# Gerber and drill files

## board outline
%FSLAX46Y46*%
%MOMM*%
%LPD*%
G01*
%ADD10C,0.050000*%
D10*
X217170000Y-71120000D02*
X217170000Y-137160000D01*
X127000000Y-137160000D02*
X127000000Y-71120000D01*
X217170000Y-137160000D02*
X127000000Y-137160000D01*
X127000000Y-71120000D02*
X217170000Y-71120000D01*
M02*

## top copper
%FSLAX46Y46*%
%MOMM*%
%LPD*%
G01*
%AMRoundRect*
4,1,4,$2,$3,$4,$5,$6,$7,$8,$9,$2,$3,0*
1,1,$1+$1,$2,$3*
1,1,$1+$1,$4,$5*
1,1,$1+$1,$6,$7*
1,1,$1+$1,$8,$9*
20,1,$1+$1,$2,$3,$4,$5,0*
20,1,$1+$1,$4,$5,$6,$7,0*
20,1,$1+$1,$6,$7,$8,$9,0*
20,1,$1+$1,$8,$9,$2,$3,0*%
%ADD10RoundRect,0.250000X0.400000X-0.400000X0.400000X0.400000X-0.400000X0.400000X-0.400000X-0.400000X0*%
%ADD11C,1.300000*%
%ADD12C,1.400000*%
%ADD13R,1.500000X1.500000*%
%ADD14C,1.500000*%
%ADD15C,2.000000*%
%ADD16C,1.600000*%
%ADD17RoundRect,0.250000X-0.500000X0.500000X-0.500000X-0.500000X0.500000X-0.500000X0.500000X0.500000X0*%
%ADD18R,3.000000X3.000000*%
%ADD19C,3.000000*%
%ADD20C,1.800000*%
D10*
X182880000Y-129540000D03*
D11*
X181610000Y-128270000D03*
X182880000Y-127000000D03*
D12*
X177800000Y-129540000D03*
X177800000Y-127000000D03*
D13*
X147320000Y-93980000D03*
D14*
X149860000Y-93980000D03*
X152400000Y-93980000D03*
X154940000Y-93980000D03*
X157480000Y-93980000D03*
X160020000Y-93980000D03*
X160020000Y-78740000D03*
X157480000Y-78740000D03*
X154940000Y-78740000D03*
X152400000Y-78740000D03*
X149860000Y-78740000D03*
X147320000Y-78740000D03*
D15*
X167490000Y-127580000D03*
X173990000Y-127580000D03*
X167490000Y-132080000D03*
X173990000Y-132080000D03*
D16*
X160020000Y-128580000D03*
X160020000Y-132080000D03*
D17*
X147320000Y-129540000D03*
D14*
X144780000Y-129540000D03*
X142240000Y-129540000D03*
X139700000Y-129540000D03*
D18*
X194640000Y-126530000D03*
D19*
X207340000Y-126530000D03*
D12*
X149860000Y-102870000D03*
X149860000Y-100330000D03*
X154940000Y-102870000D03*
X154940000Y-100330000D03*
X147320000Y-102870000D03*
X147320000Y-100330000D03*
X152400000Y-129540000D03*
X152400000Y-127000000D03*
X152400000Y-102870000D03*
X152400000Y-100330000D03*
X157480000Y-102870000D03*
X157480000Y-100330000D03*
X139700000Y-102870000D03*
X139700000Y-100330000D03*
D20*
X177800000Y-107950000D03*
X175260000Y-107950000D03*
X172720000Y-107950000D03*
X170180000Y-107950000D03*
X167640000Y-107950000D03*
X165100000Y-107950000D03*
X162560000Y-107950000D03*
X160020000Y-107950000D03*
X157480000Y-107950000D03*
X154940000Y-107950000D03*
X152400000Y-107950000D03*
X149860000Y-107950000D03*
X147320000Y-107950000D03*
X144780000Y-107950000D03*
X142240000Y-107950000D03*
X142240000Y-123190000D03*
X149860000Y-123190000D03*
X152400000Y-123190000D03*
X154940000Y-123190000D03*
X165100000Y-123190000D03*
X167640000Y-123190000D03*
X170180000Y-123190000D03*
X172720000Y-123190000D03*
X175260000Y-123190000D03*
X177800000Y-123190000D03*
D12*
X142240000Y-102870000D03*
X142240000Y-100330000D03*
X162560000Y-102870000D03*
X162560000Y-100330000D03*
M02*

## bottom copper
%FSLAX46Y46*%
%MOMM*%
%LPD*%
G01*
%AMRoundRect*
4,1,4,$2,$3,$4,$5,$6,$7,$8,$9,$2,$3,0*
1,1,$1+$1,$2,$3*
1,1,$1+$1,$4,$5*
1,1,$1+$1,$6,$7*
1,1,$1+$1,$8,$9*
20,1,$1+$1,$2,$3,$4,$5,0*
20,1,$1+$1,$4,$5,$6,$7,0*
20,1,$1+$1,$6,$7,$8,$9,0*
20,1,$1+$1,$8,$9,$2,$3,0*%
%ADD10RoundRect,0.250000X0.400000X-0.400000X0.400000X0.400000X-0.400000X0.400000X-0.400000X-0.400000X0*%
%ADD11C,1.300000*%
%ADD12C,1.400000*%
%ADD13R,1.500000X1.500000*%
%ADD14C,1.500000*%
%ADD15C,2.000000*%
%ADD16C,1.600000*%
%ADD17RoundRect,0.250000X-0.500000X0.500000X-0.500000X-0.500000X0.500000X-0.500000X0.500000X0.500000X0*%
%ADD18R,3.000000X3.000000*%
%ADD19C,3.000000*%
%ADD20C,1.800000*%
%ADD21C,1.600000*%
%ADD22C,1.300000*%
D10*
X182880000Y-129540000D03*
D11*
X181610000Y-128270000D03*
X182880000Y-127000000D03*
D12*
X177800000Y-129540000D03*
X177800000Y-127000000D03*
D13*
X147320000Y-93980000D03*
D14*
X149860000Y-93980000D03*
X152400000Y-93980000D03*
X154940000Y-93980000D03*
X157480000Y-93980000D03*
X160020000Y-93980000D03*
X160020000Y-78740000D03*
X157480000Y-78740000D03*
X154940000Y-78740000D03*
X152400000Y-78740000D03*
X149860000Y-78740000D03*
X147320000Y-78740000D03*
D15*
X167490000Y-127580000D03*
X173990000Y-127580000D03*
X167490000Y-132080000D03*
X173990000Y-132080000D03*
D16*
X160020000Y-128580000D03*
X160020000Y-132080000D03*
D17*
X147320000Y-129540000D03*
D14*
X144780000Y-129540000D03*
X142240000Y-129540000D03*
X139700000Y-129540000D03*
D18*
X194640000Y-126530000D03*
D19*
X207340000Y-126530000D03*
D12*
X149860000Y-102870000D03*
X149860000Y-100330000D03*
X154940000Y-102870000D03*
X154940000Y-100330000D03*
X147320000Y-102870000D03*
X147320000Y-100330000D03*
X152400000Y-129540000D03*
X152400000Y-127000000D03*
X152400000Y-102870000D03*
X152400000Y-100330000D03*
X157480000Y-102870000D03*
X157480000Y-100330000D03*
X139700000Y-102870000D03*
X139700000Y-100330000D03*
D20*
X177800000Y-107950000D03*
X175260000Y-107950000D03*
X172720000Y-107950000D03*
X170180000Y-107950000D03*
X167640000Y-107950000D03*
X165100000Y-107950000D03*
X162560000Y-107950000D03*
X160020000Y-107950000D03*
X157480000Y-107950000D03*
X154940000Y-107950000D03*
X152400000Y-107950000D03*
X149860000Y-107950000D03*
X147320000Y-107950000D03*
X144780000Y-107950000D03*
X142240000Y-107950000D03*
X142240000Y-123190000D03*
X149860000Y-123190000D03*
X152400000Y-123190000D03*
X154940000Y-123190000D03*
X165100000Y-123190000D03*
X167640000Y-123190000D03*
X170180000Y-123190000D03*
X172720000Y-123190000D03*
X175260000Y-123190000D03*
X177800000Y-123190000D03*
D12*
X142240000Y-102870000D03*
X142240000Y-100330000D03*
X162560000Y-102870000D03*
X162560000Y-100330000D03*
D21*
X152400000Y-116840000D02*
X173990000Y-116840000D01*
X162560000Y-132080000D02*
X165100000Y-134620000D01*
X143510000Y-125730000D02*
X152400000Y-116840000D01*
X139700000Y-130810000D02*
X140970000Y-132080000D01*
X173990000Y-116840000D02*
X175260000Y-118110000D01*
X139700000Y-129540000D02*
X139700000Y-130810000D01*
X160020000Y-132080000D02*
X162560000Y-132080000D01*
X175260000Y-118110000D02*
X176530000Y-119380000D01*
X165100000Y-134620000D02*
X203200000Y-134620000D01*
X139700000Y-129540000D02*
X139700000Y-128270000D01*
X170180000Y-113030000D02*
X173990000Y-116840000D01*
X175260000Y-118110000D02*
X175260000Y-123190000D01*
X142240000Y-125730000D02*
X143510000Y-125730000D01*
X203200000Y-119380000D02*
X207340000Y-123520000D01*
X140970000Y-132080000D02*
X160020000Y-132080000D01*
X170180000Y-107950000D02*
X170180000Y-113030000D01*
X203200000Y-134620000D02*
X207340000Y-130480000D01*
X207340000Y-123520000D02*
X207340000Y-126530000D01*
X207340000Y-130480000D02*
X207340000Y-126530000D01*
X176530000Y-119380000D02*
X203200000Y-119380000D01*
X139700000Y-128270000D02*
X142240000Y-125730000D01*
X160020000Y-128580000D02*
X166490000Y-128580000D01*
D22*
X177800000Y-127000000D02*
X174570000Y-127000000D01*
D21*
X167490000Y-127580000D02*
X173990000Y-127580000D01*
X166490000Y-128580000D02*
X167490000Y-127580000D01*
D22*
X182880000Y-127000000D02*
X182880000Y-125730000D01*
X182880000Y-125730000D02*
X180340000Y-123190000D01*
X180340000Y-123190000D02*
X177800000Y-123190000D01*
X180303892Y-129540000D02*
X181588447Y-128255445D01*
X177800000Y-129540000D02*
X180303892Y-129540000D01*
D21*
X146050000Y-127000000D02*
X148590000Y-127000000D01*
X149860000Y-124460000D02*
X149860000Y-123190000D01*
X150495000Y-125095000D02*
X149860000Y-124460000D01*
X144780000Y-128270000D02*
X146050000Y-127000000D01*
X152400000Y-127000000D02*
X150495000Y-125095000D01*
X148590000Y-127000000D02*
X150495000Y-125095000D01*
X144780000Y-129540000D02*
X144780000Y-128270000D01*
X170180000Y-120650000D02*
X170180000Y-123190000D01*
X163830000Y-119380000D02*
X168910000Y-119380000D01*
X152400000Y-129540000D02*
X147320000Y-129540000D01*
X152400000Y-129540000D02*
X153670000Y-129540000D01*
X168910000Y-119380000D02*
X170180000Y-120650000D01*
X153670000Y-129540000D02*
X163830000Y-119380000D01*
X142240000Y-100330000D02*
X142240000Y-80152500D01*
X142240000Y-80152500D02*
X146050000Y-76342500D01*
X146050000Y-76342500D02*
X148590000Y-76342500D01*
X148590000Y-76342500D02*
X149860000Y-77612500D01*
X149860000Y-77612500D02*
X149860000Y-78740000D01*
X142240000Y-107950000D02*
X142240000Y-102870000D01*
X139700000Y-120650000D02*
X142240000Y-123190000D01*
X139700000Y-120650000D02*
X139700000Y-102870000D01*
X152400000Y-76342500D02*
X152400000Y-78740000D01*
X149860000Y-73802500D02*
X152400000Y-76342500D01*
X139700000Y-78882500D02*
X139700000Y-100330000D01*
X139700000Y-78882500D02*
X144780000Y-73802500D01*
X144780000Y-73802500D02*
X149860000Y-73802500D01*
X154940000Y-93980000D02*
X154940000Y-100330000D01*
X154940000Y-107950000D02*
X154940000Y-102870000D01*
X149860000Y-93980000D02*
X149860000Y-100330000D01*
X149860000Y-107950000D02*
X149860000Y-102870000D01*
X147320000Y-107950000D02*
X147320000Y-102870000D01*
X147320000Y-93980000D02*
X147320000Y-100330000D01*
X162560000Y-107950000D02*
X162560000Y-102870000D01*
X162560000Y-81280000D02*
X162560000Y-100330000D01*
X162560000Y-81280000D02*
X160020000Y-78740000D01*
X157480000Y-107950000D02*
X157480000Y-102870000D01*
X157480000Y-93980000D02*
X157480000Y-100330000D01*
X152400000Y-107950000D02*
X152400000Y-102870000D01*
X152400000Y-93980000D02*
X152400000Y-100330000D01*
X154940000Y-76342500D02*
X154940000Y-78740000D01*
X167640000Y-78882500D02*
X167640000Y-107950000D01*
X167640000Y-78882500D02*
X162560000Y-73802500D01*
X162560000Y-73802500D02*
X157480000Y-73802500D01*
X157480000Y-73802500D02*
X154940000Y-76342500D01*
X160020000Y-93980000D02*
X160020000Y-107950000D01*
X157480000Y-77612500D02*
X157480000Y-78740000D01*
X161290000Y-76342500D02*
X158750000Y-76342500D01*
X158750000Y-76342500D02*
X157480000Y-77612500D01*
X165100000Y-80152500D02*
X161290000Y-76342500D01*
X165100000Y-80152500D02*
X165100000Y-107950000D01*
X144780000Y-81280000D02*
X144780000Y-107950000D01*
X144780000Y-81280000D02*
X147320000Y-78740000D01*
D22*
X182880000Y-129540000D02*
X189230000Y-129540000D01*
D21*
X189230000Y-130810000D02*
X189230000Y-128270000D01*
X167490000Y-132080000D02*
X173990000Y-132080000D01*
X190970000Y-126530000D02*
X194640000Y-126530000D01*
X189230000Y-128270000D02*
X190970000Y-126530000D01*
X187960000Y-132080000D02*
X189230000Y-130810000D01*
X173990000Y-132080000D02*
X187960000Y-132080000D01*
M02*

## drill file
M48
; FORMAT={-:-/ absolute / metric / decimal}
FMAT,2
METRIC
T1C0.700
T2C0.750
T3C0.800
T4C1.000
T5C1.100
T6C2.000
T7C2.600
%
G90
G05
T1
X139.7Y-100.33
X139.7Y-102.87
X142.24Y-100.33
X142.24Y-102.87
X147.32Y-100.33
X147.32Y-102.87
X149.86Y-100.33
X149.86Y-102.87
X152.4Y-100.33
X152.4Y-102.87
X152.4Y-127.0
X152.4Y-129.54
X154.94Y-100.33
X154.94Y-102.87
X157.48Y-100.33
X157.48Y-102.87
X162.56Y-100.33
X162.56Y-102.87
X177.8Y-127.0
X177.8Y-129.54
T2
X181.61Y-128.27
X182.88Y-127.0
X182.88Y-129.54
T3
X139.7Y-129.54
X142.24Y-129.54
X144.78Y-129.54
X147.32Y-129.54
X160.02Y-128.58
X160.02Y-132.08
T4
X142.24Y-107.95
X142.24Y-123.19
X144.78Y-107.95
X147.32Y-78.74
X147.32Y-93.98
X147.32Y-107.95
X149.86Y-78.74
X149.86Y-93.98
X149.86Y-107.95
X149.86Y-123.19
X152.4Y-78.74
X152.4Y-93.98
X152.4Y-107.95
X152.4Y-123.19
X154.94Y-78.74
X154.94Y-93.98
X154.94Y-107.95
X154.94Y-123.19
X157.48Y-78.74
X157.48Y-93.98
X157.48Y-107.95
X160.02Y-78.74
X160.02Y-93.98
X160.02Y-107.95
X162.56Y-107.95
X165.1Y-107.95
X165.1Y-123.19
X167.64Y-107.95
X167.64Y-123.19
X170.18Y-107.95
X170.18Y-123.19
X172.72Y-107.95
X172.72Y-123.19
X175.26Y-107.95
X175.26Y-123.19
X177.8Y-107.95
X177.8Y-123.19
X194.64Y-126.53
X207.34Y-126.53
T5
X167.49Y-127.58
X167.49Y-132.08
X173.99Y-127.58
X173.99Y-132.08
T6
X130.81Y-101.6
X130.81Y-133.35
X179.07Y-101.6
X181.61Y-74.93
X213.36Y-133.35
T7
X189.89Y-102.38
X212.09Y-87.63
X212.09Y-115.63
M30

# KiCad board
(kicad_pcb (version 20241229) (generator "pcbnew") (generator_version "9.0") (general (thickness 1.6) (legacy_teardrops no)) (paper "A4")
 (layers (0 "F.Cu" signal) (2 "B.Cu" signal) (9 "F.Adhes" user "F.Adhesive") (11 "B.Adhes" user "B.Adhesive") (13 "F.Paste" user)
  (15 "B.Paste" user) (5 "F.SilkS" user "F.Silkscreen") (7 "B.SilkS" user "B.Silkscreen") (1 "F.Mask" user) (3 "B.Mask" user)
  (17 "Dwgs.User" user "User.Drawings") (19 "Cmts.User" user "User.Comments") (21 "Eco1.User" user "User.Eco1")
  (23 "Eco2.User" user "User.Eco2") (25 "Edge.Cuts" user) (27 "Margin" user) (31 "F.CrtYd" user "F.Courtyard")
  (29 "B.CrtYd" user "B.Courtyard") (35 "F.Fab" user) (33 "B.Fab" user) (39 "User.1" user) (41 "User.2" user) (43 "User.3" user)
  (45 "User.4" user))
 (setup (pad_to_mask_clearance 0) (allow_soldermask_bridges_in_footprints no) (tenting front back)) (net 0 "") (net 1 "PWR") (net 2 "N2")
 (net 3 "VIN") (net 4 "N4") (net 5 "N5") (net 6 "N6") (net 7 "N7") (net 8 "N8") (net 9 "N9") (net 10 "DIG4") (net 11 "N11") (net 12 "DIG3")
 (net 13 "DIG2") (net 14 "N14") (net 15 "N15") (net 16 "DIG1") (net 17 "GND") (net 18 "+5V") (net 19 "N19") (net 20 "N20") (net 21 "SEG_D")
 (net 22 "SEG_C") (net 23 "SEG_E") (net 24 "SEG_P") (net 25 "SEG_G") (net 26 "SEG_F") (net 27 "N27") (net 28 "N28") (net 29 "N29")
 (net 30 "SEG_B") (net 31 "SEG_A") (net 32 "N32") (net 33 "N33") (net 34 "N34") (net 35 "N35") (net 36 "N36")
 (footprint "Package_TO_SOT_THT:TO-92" (layer "F.Cu") (at 182.88 129.54 90)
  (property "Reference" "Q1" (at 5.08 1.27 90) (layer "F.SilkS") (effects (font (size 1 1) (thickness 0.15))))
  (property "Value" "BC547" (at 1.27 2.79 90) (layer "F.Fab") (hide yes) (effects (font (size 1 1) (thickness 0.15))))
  (pad "1" thru_hole roundrect (at 0 0 90) (size 1.3 1.3) (drill 0.75) (layers "*.Cu" "*.Mask") (remove_unused_layers no)
   (roundrect_rratio 0.1923076923) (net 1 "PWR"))
  (pad "2" thru_hole circle (at 1.27 -1.27 90) (size 1.3 1.3) (drill 0.75) (layers "*.Cu" "*.Mask") (remove_unused_layers no) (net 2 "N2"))
  (pad "3" thru_hole circle (at 2.54 0 90) (size 1.3 1.3) (drill 0.75) (layers "*.Cu" "*.Mask") (remove_unused_layers no) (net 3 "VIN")))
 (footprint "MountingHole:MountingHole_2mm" (layer "F.Cu") (at 130.81 133.35)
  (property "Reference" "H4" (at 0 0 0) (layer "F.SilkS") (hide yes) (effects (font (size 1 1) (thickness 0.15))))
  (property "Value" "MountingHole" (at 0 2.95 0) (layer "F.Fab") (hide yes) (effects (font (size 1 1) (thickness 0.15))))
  (pad "" np_thru_hole circle (at 0 0) (size 2 2) (drill 2) (layers "*.Cu" "*.Mask")))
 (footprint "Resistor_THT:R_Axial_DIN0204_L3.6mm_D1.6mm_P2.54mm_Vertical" (layer "F.Cu") (at 177.8 129.54 90)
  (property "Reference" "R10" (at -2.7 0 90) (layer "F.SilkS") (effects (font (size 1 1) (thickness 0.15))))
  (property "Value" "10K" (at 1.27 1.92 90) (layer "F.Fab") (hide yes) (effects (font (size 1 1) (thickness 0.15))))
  (pad "1" thru_hole circle (at 0 0 90) (size 1.4 1.4) (drill 0.7) (layers "*.Cu" "*.Mask") (remove_unused_layers no) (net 2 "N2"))
  (pad "2" thru_hole circle (at 2.54 0 90) (size 1.4 1.4) (drill 0.7) (layers "*.Cu" "*.Mask") (remove_unused_layers no) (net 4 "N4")))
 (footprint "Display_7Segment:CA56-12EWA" (layer "F.Cu") (at 147.32 93.98 90)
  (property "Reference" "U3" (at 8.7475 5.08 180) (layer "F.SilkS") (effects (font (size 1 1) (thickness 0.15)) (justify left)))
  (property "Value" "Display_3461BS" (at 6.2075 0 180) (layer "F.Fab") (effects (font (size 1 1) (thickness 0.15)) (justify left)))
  (pad "1" thru_hole rect (at 0 0 90) (size 1.5 1.5) (drill 1) (layers "*.Cu" "*.Mask") (remove_unused_layers no) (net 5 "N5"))
  (pad "2" thru_hole circle (at 0 2.54 90) (size 1.5 1.5) (drill 1) (layers "*.Cu" "*.Mask") (remove_unused_layers no) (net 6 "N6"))
  (pad "3" thru_hole circle (at 0 5.08 90) (size 1.5 1.5) (drill 1) (layers "*.Cu" "*.Mask") (remove_unused_layers no) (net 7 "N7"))
  (pad "4" thru_hole circle (at 0 7.62 90) (size 1.5 1.5) (drill 1) (layers "*.Cu" "*.Mask") (remove_unused_layers no) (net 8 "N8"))
  (pad "5" thru_hole circle (at 0 10.16 90) (size 1.5 1.5) (drill 1) (layers "*.Cu" "*.Mask") (remove_unused_layers no) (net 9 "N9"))
  (pad "6" thru_hole circle (at 0 12.7 90) (size 1.5 1.5) (drill 1) (layers "*.Cu" "*.Mask") (remove_unused_layers no) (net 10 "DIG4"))
  (pad "7" thru_hole circle (at 15.24 12.7 90) (size 1.5 1.5) (drill 1) (layers "*.Cu" "*.Mask") (remove_unused_layers no) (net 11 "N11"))
  (pad "8" thru_hole circle (at 15.24 10.16 90) (size 1.5 1.5) (drill 1) (layers "*.Cu" "*.Mask") (remove_unused_layers no) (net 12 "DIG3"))
  (pad "9" thru_hole circle (at 15.24 7.62 90) (size 1.5 1.5) (drill 1) (layers "*.Cu" "*.Mask") (remove_unused_layers no) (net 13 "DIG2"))
  (pad "10" thru_hole circle (at 15.24 5.08 90) (size 1.5 1.5) (drill 1) (layers "*.Cu" "*.Mask") (remove_unused_layers no) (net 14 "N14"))
  (pad "11" thru_hole circle (at 15.24 2.54 90) (size 1.5 1.5) (drill 1) (layers "*.Cu" "*.Mask") (remove_unused_layers no) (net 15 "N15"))
  (pad "12" thru_hole circle (at 15.24 0 90) (size 1.5 1.5) (drill 1) (layers "*.Cu" "*.Mask") (remove_unused_layers no) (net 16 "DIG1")))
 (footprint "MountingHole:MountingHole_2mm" (layer "F.Cu") (at 130.81 101.6)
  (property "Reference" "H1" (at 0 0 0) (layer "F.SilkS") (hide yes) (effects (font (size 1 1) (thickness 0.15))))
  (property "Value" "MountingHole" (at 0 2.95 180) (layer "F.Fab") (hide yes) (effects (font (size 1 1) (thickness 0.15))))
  (pad "" np_thru_hole circle (at 0 0) (size 2 2) (drill 2) (layers "*.Cu" "*.Mask")))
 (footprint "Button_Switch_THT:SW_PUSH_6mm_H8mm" (layer "F.Cu") (at 167.49 127.58)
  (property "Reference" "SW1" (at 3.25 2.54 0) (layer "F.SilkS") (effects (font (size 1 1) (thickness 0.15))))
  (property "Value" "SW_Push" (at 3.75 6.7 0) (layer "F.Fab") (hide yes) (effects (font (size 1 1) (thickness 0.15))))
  (pad "1" thru_hole circle (at 0 0 90) (size 2 2) (drill 1.1) (layers "*.Cu" "*.Mask") (remove_unused_layers no) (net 4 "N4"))
  (pad "1" thru_hole circle (at 6.5 0 90) (size 2 2) (drill 1.1) (layers "*.Cu" "*.Mask") (remove_unused_layers no) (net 4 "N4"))
  (pad "2" thru_hole circle (at 0 4.5 90) (size 2 2) (drill 1.1) (layers "*.Cu" "*.Mask") (remove_unused_layers no) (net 1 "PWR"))
  (pad "2" thru_hole circle (at 6.5 4.5 90) (size 2 2) (drill 1.1) (layers "*.Cu" "*.Mask") (remove_unused_layers no) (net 1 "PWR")))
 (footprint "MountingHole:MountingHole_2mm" (layer "F.Cu") (at 179.07 101.6)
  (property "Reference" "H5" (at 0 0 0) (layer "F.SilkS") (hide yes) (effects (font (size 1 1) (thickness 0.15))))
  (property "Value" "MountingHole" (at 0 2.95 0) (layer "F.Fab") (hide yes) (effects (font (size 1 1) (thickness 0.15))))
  (pad "" np_thru_hole circle (at 0 0) (size 2 2) (drill 2) (layers "*.Cu" "*.Mask")))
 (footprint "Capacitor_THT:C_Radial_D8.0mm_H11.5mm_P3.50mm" (layer "F.Cu") (at 160.02 128.58 -90)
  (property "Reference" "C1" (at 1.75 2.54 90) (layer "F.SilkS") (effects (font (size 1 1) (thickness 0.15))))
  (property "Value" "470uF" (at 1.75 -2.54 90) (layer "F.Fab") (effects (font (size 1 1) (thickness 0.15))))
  (pad "1" thru_hole circle (at 0 0 270) (size 1.6 1.6) (drill 0.8) (layers "*.Cu" "*.Mask") (remove_unused_layers no) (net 4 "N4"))
  (pad "2" thru_hole circle (at 3.5 0 270) (size 1.6 1.6) (drill 0.8) (layers "*.Cu" "*.Mask") (remove_unused_layers no) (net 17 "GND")))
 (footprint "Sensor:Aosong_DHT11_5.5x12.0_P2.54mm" (layer "F.Cu") (at 147.32 129.54 -90)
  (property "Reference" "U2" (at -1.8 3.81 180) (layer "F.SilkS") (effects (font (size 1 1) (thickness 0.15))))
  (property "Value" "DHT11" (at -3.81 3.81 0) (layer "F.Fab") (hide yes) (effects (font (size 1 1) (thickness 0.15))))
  (pad "1" thru_hole roundrect (at 0 0 270) (size 1.5 1.5) (drill 0.8) (layers "*.Cu" "*.Mask") (remove_unused_layers no)
   (roundrect_rratio 0.1666666667) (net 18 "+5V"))
  (pad "2" thru_hole circle (at 0 2.54 270) (size 1.5 1.5) (drill 0.8) (layers "*.Cu" "*.Mask") (remove_unused_layers no) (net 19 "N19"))
  (pad "3" thru_hole circle (at 0 5.08 270) (size 1.5 1.5) (drill 0.8) (layers "*.Cu" "*.Mask") (remove_unused_layers no) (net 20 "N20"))
  (pad "4" thru_hole circle (at 0 7.62 270) (size 1.5 1.5) (drill 0.8) (layers "*.Cu" "*.Mask") (remove_unused_layers no) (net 17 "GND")))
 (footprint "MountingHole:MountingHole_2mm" (layer "F.Cu") (at 213.36 133.35)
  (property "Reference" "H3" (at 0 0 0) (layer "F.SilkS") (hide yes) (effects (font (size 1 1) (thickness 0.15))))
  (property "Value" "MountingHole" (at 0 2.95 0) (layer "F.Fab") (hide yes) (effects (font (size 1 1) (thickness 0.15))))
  (pad "" np_thru_hole circle (at 0 0) (size 2 2) (drill 2) (layers "*.Cu" "*.Mask")))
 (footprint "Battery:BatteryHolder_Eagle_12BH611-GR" (layer "F.Cu") (at 194.64 126.53 -90)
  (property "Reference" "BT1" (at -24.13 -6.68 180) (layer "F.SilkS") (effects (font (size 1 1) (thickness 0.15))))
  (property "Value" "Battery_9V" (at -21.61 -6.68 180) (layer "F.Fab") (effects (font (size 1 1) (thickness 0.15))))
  (pad "" np_thru_hole circle (at -38.9 -17.45 270) (size 2.6 2.6) (drill 2.6) (layers "*.Cu" "*.Mask"))
  (pad "" np_thru_hole circle (at -24.15 4.75 270) (size 2.6 2.6) (drill 2.6) (layers "*.Cu" "*.Mask"))
  (pad "" np_thru_hole circle (at -10.9 -17.45 270) (size 2.6 2.6) (drill 2.6) (layers "*.Cu" "*.Mask"))
  (pad "1" thru_hole rect (at 0 0 270) (size 3 3) (drill 1) (layers "*.Cu" "*.Mask") (remove_unused_layers no) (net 1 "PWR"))
  (pad "2" thru_hole circle (at 0 -12.7 270) (size 3 3) (drill 1) (layers "*.Cu" "*.Mask") (remove_unused_layers no) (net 17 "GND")))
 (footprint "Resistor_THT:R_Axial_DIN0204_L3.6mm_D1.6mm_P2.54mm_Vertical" (layer "F.Cu") (at 149.86 102.87 90)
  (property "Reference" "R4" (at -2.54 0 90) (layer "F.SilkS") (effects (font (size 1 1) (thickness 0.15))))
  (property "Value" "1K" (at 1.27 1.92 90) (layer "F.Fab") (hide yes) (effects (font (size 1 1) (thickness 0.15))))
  (pad "1" thru_hole circle (at 0 0 90) (size 1.4 1.4) (drill 0.7) (layers "*.Cu" "*.Mask") (remove_unused_layers no) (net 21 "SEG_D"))
  (pad "2" thru_hole circle (at 2.54 0 90) (size 1.4 1.4) (drill 0.7) (layers "*.Cu" "*.Mask") (remove_unused_layers no) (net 6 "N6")))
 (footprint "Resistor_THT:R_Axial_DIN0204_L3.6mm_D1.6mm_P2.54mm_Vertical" (layer "F.Cu") (at 154.94 102.87 90)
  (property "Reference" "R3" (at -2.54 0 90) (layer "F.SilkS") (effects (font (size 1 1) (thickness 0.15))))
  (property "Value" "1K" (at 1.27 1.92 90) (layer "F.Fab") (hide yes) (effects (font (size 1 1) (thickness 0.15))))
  (pad "1" thru_hole circle (at 0 0 90) (size 1.4 1.4) (drill 0.7) (layers "*.Cu" "*.Mask") (remove_unused_layers no) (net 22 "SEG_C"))
  (pad "2" thru_hole circle (at 2.54 0 90) (size 1.4 1.4) (drill 0.7) (layers "*.Cu" "*.Mask") (remove_unused_layers no) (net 8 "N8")))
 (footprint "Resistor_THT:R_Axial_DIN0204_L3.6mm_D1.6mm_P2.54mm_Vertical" (layer "F.Cu") (at 147.32 102.87 90)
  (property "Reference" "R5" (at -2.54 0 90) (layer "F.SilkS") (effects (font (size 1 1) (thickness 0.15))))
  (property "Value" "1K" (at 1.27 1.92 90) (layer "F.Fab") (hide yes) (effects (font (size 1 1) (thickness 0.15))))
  (pad "1" thru_hole circle (at 0 0 90) (size 1.4 1.4) (drill 0.7) (layers "*.Cu" "*.Mask") (remove_unused_layers no) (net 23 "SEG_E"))
  (pad "2" thru_hole circle (at 2.54 0 90) (size 1.4 1.4) (drill 0.7) (layers "*.Cu" "*.Mask") (remove_unused_layers no) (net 5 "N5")))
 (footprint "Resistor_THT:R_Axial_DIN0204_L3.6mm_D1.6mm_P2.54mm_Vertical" (layer "F.Cu") (at 152.4 129.54 90)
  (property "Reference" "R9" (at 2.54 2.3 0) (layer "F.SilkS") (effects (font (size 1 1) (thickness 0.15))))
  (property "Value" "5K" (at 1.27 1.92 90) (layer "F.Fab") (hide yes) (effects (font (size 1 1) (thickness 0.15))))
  (pad "1" thru_hole circle (at 0 0 90) (size 1.4 1.4) (drill 0.7) (layers "*.Cu" "*.Mask") (remove_unused_layers no) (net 18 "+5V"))
  (pad "2" thru_hole circle (at 2.54 0 90) (size 1.4 1.4) (drill 0.7) (layers "*.Cu" "*.Mask") (remove_unused_layers no) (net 19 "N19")))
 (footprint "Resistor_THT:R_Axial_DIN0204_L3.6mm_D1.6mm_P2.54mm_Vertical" (layer "F.Cu") (at 152.4 102.87 90)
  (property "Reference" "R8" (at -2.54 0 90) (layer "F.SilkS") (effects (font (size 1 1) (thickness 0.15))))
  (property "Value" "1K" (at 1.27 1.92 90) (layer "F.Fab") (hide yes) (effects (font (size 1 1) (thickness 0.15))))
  (pad "1" thru_hole circle (at 0 0 90) (size 1.4 1.4) (drill 0.7) (layers "*.Cu" "*.Mask") (remove_unused_layers no) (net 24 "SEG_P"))
  (pad "2" thru_hole circle (at 2.54 0 90) (size 1.4 1.4) (drill 0.7) (layers "*.Cu" "*.Mask") (remove_unused_layers no) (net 7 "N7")))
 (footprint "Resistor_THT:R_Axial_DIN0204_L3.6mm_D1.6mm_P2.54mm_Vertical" (layer "F.Cu") (at 157.48 102.87 90)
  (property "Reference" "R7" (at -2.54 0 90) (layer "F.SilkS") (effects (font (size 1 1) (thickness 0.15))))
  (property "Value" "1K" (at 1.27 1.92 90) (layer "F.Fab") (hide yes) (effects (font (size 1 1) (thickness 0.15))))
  (pad "1" thru_hole circle (at 0 0 90) (size 1.4 1.4) (drill 0.7) (layers "*.Cu" "*.Mask") (remove_unused_layers no) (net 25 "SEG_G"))
  (pad "2" thru_hole circle (at 2.54 0 90) (size 1.4 1.4) (drill 0.7) (layers "*.Cu" "*.Mask") (remove_unused_layers no) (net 9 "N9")))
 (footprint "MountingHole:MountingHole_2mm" (layer "F.Cu") (at 181.61 74.93)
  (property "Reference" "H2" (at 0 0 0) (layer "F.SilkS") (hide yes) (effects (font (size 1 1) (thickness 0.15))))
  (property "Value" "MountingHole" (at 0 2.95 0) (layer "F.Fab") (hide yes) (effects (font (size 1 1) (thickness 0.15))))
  (pad "" np_thru_hole circle (at 0 0) (size 2 2) (drill 2) (layers "*.Cu" "*.Mask")))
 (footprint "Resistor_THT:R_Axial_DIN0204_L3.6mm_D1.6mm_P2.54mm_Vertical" (layer "F.Cu") (at 139.7 102.87 90)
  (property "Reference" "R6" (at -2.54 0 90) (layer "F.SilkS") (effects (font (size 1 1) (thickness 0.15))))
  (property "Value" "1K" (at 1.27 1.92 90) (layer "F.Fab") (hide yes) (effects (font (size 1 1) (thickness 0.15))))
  (pad "1" thru_hole circle (at 0 0 90) (size 1.4 1.4) (drill 0.7) (layers "*.Cu" "*.Mask") (remove_unused_layers no) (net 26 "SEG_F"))
  (pad "2" thru_hole circle (at 2.54 0 90) (size 1.4 1.4) (drill 0.7) (layers "*.Cu" "*.Mask") (remove_unused_layers no) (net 14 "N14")))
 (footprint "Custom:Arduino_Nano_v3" (layer "F.Cu") (at 177.8 107.95 -90)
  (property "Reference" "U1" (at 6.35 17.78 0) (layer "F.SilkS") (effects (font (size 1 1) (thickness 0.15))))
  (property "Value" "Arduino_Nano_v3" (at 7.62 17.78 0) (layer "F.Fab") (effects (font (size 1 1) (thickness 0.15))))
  (pad "1" thru_hole circle (at 0 0 270) (size 1.8 1.8) (drill 1) (layers "*.Cu" "*.Mask") (remove_unused_layers no) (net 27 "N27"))
  (pad "2" thru_hole circle (at 0 2.54 270) (size 1.8 1.8) (drill 1) (layers "*.Cu" "*.Mask") (remove_unused_layers no) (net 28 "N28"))
  (pad "3" thru_hole circle (at 0 5.08 270) (size 1.8 1.8) (drill 1) (layers "*.Cu" "*.Mask") (remove_unused_layers no) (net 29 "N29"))
  (pad "4" thru_hole circle (at 0 7.62 270) (size 1.8 1.8) (drill 1) (layers "*.Cu" "*.Mask") (remove_unused_layers no) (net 17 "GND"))
  (pad "5" thru_hole circle (at 0 10.16 270) (size 1.8 1.8) (drill 1) (layers "*.Cu" "*.Mask") (remove_unused_layers no) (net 13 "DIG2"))
  (pad "6" thru_hole circle (at 0 12.7 270) (size 1.8 1.8) (drill 1) (layers "*.Cu" "*.Mask") (remove_unused_layers no) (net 12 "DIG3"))
  (pad "7" thru_hole circle (at 0 15.24 270) (size 1.8 1.8) (drill 1) (layers "*.Cu" "*.Mask") (remove_unused_layers no) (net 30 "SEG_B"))
  (pad "8" thru_hole circle (at 0 17.78 270) (size 1.8 1.8) (drill 1) (layers "*.Cu" "*.Mask") (remove_unused_layers no) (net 10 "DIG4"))
  (pad "9" thru_hole circle (at 0 20.32 270) (size 1.8 1.8) (drill 1) (layers "*.Cu" "*.Mask") (remove_unused_layers no) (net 25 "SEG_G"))
  (pad "10" thru_hole circle (at 0 22.86 270) (size 1.8 1.8) (drill 1) (layers "*.Cu" "*.Mask") (remove_unused_layers no) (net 22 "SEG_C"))
  (pad "11" thru_hole circle (at 0 25.4 270) (size 1.8 1.8) (drill 1) (layers "*.Cu" "*.Mask") (remove_unused_layers no) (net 24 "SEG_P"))
  (pad "12" thru_hole circle (at 0 27.94 270) (size 1.8 1.8) (drill 1) (layers "*.Cu" "*.Mask") (remove_unused_layers no) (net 21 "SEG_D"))
  (pad "13" thru_hole circle (at 0 30.48 270) (size 1.8 1.8) (drill 1) (layers "*.Cu" "*.Mask") (remove_unused_layers no) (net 23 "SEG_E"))
  (pad "14" thru_hole circle (at 0 33.02 270) (size 1.8 1.8) (drill 1) (layers "*.Cu" "*.Mask") (remove_unused_layers no) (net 16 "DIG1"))
  (pad "15" thru_hole circle (at 0 35.56 270) (size 1.8 1.8) (drill 1) (layers "*.Cu" "*.Mask") (remove_unused_layers no) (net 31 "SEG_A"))
  (pad "16" thru_hole circle (at 15.24 35.56 270) (size 1.8 1.8) (drill 1) (layers "*.Cu" "*.Mask") (remove_unused_layers no)
   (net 26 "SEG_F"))
  (pad "19" thru_hole circle (at 15.24 27.94 270) (size 1.8 1.8) (drill 1) (layers "*.Cu" "*.Mask") (remove_unused_layers no) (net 19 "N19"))
  (pad "20" thru_hole circle (at 15.24 25.4 270) (size 1.8 1.8) (drill 1) (layers "*.Cu" "*.Mask") (remove_unused_layers no) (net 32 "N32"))
  (pad "21" thru_hole circle (at 15.24 22.86 270) (size 1.8 1.8) (drill 1) (layers "*.Cu" "*.Mask") (remove_unused_layers no) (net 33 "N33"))
  (pad "25" thru_hole circle (at 15.24 12.7 270) (size 1.8 1.8) (drill 1) (layers "*.Cu" "*.Mask") (remove_unused_layers no) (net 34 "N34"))
  (pad "26" thru_hole circle (at 15.24 10.16 270) (size 1.8 1.8) (drill 1) (layers "*.Cu" "*.Mask") (remove_unused_layers no) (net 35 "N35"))
  (pad "27" thru_hole circle (at 15.24 7.62 270) (size 1.8 1.8) (drill 1) (layers "*.Cu" "*.Mask") (remove_unused_layers no) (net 18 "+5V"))
  (pad "28" thru_hole circle (at 15.24 5.08 270) (size 1.8 1.8) (drill 1) (layers "*.Cu" "*.Mask") (remove_unused_layers no) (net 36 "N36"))
  (pad "29" thru_hole circle (at 15.24 2.54 270) (size 1.8 1.8) (drill 1) (layers "*.Cu" "*.Mask") (remove_unused_layers no) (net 17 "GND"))
  (pad "30" thru_hole circle (at 15.24 0 270) (size 1.8 1.8) (drill 1) (layers "*.Cu" "*.Mask") (remove_unused_layers no) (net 3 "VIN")))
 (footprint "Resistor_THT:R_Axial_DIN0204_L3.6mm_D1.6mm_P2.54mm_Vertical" (layer "F.Cu") (at 142.24 102.87 90)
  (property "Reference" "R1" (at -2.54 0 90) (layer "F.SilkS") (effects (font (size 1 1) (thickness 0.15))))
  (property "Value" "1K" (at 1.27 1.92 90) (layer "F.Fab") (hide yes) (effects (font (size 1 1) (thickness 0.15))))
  (pad "1" thru_hole circle (at 0 0 90) (size 1.4 1.4) (drill 0.7) (layers "*.Cu" "*.Mask") (remove_unused_layers no) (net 31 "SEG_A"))
  (pad "2" thru_hole circle (at 2.54 0 90) (size 1.4 1.4) (drill 0.7) (layers "*.Cu" "*.Mask") (remove_unused_layers no) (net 15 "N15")))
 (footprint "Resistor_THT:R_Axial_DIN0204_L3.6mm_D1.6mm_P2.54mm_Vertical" (layer "F.Cu") (at 162.56 102.87 90)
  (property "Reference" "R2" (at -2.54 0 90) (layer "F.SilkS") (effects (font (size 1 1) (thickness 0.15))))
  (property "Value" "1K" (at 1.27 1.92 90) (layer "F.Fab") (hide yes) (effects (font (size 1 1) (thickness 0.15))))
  (pad "1" thru_hole circle (at 0 0 90) (size 1.4 1.4) (drill 0.7) (layers "*.Cu" "*.Mask") (remove_unused_layers no) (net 30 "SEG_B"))
  (pad "2" thru_hole circle (at 2.54 0 90) (size 1.4 1.4) (drill 0.7) (layers "*.Cu" "*.Mask") (remove_unused_layers no) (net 11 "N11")))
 (gr_line (start 217.17 71.12) (end 217.17 137.16) (stroke (width 0.05) (type default)) (layer "Edge.Cuts"))
 (gr_line (start 127 137.16) (end 127 71.12) (stroke (width 0.05) (type default)) (layer "Edge.Cuts"))
 (gr_line (start 217.17 137.16) (end 127 137.16) (stroke (width 0.05) (type default)) (layer "Edge.Cuts"))
 (gr_line (start 127 71.12) (end 217.17 71.12) (stroke (width 0.05) (type default)) (layer "Edge.Cuts"))
 (segment (start 152.4 116.84) (end 173.99 116.84) (width 1.6) (layer "B.Cu") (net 17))
 (segment (start 162.56 132.08) (end 165.1 134.62) (width 1.6) (layer "B.Cu") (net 17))
 (segment (start 143.51 125.73) (end 152.4 116.84) (width 1.6) (layer "B.Cu") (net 17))
 (segment (start 139.7 130.81) (end 140.97 132.08) (width 1.6) (layer "B.Cu") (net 17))
 (segment (start 173.99 116.84) (end 175.26 118.11) (width 1.6) (layer "B.Cu") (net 17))
 (segment (start 139.7 129.54) (end 139.7 130.81) (width 1.6) (layer "B.Cu") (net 17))
 (segment (start 160.02 132.08) (end 162.56 132.08) (width 1.6) (layer "B.Cu") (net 17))
 (segment (start 175.26 118.11) (end 176.53 119.38) (width 1.6) (layer "B.Cu") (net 17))
 (segment (start 165.1 134.62) (end 203.2 134.62) (width 1.6) (layer "B.Cu") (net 17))
 (segment (start 139.7 129.54) (end 139.7 128.27) (width 1.6) (layer "B.Cu") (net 17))
 (segment (start 170.18 113.03) (end 173.99 116.84) (width 1.6) (layer "B.Cu") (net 17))
 (segment (start 175.26 118.11) (end 175.26 123.19) (width 1.6) (layer "B.Cu") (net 17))
 (segment (start 142.24 125.73) (end 143.51 125.73) (width 1.6) (layer "B.Cu") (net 17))
 (segment (start 203.2 119.38) (end 207.34 123.52) (width 1.6) (layer "B.Cu") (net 17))
 (segment (start 140.97 132.08) (end 160.02 132.08) (width 1.6) (layer "B.Cu") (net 17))
 (segment (start 170.18 107.95) (end 170.18 113.03) (width 1.6) (layer "B.Cu") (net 17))
 (segment (start 203.2 134.62) (end 207.34 130.48) (width 1.6) (layer "B.Cu") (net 17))
 (segment (start 207.34 123.52) (end 207.34 126.53) (width 1.6) (layer "B.Cu") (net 17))
 (segment (start 207.34 130.48) (end 207.34 126.53) (width 1.6) (layer "B.Cu") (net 17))
 (segment (start 176.53 119.38) (end 203.2 119.38) (width 1.6) (layer "B.Cu") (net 17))
 (segment (start 139.7 128.27) (end 142.24 125.73) (width 1.6) (layer "B.Cu") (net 17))
 (segment (start 160.02 128.58) (end 166.49 128.58) (width 1.6) (layer "B.Cu") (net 4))
 (segment (start 177.8 127) (end 174.57 127) (width 1.3) (layer "B.Cu") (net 4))
 (segment (start 167.49 127.58) (end 173.99 127.58) (width 1.6) (layer "B.Cu") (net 4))
 (segment (start 166.49 128.58) (end 167.49 127.58) (width 1.6) (layer "B.Cu") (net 4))
 (segment (start 182.88 127) (end 182.88 125.73) (width 1.3) (layer "B.Cu") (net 3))
 (segment (start 182.88 125.73) (end 180.34 123.19) (width 1.3) (layer "B.Cu") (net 3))
 (segment (start 180.34 123.19) (end 177.8 123.19) (width 1.3) (layer "B.Cu") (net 3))
 (segment (start 180.303892 129.54) (end 181.588447 128.255445) (width 1.3) (layer "B.Cu") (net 2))
 (segment (start 177.8 129.54) (end 180.303892 129.54) (width 1.3) (layer "B.Cu") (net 2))
 (segment (start 146.05 127) (end 148.59 127) (width 1.6) (layer "B.Cu") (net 19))
 (segment (start 149.86 124.46) (end 149.86 123.19) (width 1.6) (layer "B.Cu") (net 19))
 (segment (start 150.495 125.095) (end 149.86 124.46) (width 1.6) (layer "B.Cu") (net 19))
 (segment (start 144.78 128.27) (end 146.05 127) (width 1.6) (layer "B.Cu") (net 19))
 (segment (start 152.4 127) (end 150.495 125.095) (width 1.6) (layer "B.Cu") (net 19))
 (segment (start 148.59 127) (end 150.495 125.095) (width 1.6) (layer "B.Cu") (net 19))
 (segment (start 144.78 129.54) (end 144.78 128.27) (width 1.6) (layer "B.Cu") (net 19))
 (segment (start 170.18 120.65) (end 170.18 123.19) (width 1.6) (layer "B.Cu") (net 18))
 (segment (start 163.83 119.38) (end 168.91 119.38) (width 1.6) (layer "B.Cu") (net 18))
 (segment (start 152.4 129.54) (end 147.32 129.54) (width 1.6) (layer "B.Cu") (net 18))
 (segment (start 152.4 129.54) (end 153.67 129.54) (width 1.6) (layer "B.Cu") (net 18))
 (segment (start 168.91 119.38) (end 170.18 120.65) (width 1.6) (layer "B.Cu") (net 18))
 (segment (start 153.67 129.54) (end 163.83 119.38) (width 1.6) (layer "B.Cu") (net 18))
 (segment (start 142.24 100.33) (end 142.24 80.1525) (width 1.6) (layer "B.Cu") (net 15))
 (segment (start 142.24 80.1525) (end 146.05 76.3425) (width 1.6) (layer "B.Cu") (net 15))
 (segment (start 146.05 76.3425) (end 148.59 76.3425) (width 1.6) (layer "B.Cu") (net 15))
 (segment (start 148.59 76.3425) (end 149.86 77.6125) (width 1.6) (layer "B.Cu") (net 15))
 (segment (start 149.86 77.6125) (end 149.86 78.74) (width 1.6) (layer "B.Cu") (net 15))
 (segment (start 142.24 107.95) (end 142.24 102.87) (width 1.6) (layer "B.Cu") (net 31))
 (segment (start 139.7 120.65) (end 142.24 123.19) (width 1.6) (layer "B.Cu") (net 26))
 (segment (start 139.7 120.65) (end 139.7 102.87) (width 1.6) (layer "B.Cu") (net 26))
 (segment (start 152.4 76.3425) (end 152.4 78.74) (width 1.6) (layer "B.Cu") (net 14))
 (segment (start 149.86 73.8025) (end 152.4 76.3425) (width 1.6) (layer "B.Cu") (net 14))
 (segment (start 139.7 78.8825) (end 139.7 100.33) (width 1.6) (layer "B.Cu") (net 14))
 (segment (start 139.7 78.8825) (end 144.78 73.8025) (width 1.6) (layer "B.Cu") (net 14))
 (segment (start 144.78 73.8025) (end 149.86 73.8025) (width 1.6) (layer "B.Cu") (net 14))
 (segment (start 154.94 93.98) (end 154.94 100.33) (width 1.6) (layer "B.Cu") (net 8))
 (segment (start 154.94 107.95) (end 154.94 102.87) (width 1.6) (layer "B.Cu") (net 22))
 (segment (start 149.86 93.98) (end 149.86 100.33) (width 1.6) (layer "B.Cu") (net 6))
 (segment (start 149.86 107.95) (end 149.86 102.87) (width 1.6) (layer "B.Cu") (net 21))
 (segment (start 147.32 107.95) (end 147.32 102.87) (width 1.6) (layer "B.Cu") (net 23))
 (segment (start 147.32 93.98) (end 147.32 100.33) (width 1.6) (layer "B.Cu") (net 5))
 (segment (start 162.56 107.95) (end 162.56 102.87) (width 1.6) (layer "B.Cu") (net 30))
 (segment (start 162.56 81.28) (end 162.56 100.33) (width 1.6) (layer "B.Cu") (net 11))
 (segment (start 162.56 81.28) (end 160.02 78.74) (width 1.6) (layer "B.Cu") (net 11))
 (segment (start 157.48 107.95) (end 157.48 102.87) (width 1.6) (layer "B.Cu") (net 25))
 (segment (start 157.48 93.98) (end 157.48 100.33) (width 1.6) (layer "B.Cu") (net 9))
 (segment (start 152.4 107.95) (end 152.4 102.87) (width 1.6) (layer "B.Cu") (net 24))
 (segment (start 152.4 93.98) (end 152.4 100.33) (width 1.6) (layer "B.Cu") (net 7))
 (segment (start 154.94 76.3425) (end 154.94 78.74) (width 1.6) (layer "B.Cu") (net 13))
 (segment (start 167.64 78.8825) (end 167.64 107.95) (width 1.6) (layer "B.Cu") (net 13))
 (segment (start 167.64 78.8825) (end 162.56 73.8025) (width 1.6) (layer "B.Cu") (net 13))
 (segment (start 162.56 73.8025) (end 157.48 73.8025) (width 1.6) (layer "B.Cu") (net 13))
 (segment (start 157.48 73.8025) (end 154.94 76.3425) (width 1.6) (layer "B.Cu") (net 13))
 (segment (start 160.02 93.98) (end 160.02 107.95) (width 1.6) (layer "B.Cu") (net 10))
 (segment (start 157.48 77.6125) (end 157.48 78.74) (width 1.6) (layer "B.Cu") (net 12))
 (segment (start 161.29 76.3425) (end 158.75 76.3425) (width 1.6) (layer "B.Cu") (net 12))
 (segment (start 158.75 76.3425) (end 157.48 77.6125) (width 1.6) (layer "B.Cu") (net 12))
 (segment (start 165.1 80.1525) (end 161.29 76.3425) (width 1.6) (layer "B.Cu") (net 12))
 (segment (start 165.1 80.1525) (end 165.1 107.95) (width 1.6) (layer "B.Cu") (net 12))
 (segment (start 144.78 81.28) (end 144.78 107.95) (width 1.6) (layer "B.Cu") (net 16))
 (segment (start 144.78 81.28) (end 147.32 78.74) (width 1.6) (layer "B.Cu") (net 16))
 (segment (start 182.88 129.54) (end 189.23 129.54) (width 1.3) (layer "B.Cu") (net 1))
 (segment (start 189.23 130.81) (end 189.23 128.27) (width 1.6) (layer "B.Cu") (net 1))
 (segment (start 167.49 132.08) (end 173.99 132.08) (width 1.6) (layer "B.Cu") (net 1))
 (segment (start 190.97 126.53) (end 194.64 126.53) (width 1.6) (layer "B.Cu") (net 1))
 (segment (start 189.23 128.27) (end 190.97 126.53) (width 1.6) (layer "B.Cu") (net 1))
 (segment (start 187.96 132.08) (end 189.23 130.81) (width 1.6) (layer "B.Cu") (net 1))
 (segment (start 173.99 132.08) (end 187.96 132.08) (width 1.6) (layer "B.Cu") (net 1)))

